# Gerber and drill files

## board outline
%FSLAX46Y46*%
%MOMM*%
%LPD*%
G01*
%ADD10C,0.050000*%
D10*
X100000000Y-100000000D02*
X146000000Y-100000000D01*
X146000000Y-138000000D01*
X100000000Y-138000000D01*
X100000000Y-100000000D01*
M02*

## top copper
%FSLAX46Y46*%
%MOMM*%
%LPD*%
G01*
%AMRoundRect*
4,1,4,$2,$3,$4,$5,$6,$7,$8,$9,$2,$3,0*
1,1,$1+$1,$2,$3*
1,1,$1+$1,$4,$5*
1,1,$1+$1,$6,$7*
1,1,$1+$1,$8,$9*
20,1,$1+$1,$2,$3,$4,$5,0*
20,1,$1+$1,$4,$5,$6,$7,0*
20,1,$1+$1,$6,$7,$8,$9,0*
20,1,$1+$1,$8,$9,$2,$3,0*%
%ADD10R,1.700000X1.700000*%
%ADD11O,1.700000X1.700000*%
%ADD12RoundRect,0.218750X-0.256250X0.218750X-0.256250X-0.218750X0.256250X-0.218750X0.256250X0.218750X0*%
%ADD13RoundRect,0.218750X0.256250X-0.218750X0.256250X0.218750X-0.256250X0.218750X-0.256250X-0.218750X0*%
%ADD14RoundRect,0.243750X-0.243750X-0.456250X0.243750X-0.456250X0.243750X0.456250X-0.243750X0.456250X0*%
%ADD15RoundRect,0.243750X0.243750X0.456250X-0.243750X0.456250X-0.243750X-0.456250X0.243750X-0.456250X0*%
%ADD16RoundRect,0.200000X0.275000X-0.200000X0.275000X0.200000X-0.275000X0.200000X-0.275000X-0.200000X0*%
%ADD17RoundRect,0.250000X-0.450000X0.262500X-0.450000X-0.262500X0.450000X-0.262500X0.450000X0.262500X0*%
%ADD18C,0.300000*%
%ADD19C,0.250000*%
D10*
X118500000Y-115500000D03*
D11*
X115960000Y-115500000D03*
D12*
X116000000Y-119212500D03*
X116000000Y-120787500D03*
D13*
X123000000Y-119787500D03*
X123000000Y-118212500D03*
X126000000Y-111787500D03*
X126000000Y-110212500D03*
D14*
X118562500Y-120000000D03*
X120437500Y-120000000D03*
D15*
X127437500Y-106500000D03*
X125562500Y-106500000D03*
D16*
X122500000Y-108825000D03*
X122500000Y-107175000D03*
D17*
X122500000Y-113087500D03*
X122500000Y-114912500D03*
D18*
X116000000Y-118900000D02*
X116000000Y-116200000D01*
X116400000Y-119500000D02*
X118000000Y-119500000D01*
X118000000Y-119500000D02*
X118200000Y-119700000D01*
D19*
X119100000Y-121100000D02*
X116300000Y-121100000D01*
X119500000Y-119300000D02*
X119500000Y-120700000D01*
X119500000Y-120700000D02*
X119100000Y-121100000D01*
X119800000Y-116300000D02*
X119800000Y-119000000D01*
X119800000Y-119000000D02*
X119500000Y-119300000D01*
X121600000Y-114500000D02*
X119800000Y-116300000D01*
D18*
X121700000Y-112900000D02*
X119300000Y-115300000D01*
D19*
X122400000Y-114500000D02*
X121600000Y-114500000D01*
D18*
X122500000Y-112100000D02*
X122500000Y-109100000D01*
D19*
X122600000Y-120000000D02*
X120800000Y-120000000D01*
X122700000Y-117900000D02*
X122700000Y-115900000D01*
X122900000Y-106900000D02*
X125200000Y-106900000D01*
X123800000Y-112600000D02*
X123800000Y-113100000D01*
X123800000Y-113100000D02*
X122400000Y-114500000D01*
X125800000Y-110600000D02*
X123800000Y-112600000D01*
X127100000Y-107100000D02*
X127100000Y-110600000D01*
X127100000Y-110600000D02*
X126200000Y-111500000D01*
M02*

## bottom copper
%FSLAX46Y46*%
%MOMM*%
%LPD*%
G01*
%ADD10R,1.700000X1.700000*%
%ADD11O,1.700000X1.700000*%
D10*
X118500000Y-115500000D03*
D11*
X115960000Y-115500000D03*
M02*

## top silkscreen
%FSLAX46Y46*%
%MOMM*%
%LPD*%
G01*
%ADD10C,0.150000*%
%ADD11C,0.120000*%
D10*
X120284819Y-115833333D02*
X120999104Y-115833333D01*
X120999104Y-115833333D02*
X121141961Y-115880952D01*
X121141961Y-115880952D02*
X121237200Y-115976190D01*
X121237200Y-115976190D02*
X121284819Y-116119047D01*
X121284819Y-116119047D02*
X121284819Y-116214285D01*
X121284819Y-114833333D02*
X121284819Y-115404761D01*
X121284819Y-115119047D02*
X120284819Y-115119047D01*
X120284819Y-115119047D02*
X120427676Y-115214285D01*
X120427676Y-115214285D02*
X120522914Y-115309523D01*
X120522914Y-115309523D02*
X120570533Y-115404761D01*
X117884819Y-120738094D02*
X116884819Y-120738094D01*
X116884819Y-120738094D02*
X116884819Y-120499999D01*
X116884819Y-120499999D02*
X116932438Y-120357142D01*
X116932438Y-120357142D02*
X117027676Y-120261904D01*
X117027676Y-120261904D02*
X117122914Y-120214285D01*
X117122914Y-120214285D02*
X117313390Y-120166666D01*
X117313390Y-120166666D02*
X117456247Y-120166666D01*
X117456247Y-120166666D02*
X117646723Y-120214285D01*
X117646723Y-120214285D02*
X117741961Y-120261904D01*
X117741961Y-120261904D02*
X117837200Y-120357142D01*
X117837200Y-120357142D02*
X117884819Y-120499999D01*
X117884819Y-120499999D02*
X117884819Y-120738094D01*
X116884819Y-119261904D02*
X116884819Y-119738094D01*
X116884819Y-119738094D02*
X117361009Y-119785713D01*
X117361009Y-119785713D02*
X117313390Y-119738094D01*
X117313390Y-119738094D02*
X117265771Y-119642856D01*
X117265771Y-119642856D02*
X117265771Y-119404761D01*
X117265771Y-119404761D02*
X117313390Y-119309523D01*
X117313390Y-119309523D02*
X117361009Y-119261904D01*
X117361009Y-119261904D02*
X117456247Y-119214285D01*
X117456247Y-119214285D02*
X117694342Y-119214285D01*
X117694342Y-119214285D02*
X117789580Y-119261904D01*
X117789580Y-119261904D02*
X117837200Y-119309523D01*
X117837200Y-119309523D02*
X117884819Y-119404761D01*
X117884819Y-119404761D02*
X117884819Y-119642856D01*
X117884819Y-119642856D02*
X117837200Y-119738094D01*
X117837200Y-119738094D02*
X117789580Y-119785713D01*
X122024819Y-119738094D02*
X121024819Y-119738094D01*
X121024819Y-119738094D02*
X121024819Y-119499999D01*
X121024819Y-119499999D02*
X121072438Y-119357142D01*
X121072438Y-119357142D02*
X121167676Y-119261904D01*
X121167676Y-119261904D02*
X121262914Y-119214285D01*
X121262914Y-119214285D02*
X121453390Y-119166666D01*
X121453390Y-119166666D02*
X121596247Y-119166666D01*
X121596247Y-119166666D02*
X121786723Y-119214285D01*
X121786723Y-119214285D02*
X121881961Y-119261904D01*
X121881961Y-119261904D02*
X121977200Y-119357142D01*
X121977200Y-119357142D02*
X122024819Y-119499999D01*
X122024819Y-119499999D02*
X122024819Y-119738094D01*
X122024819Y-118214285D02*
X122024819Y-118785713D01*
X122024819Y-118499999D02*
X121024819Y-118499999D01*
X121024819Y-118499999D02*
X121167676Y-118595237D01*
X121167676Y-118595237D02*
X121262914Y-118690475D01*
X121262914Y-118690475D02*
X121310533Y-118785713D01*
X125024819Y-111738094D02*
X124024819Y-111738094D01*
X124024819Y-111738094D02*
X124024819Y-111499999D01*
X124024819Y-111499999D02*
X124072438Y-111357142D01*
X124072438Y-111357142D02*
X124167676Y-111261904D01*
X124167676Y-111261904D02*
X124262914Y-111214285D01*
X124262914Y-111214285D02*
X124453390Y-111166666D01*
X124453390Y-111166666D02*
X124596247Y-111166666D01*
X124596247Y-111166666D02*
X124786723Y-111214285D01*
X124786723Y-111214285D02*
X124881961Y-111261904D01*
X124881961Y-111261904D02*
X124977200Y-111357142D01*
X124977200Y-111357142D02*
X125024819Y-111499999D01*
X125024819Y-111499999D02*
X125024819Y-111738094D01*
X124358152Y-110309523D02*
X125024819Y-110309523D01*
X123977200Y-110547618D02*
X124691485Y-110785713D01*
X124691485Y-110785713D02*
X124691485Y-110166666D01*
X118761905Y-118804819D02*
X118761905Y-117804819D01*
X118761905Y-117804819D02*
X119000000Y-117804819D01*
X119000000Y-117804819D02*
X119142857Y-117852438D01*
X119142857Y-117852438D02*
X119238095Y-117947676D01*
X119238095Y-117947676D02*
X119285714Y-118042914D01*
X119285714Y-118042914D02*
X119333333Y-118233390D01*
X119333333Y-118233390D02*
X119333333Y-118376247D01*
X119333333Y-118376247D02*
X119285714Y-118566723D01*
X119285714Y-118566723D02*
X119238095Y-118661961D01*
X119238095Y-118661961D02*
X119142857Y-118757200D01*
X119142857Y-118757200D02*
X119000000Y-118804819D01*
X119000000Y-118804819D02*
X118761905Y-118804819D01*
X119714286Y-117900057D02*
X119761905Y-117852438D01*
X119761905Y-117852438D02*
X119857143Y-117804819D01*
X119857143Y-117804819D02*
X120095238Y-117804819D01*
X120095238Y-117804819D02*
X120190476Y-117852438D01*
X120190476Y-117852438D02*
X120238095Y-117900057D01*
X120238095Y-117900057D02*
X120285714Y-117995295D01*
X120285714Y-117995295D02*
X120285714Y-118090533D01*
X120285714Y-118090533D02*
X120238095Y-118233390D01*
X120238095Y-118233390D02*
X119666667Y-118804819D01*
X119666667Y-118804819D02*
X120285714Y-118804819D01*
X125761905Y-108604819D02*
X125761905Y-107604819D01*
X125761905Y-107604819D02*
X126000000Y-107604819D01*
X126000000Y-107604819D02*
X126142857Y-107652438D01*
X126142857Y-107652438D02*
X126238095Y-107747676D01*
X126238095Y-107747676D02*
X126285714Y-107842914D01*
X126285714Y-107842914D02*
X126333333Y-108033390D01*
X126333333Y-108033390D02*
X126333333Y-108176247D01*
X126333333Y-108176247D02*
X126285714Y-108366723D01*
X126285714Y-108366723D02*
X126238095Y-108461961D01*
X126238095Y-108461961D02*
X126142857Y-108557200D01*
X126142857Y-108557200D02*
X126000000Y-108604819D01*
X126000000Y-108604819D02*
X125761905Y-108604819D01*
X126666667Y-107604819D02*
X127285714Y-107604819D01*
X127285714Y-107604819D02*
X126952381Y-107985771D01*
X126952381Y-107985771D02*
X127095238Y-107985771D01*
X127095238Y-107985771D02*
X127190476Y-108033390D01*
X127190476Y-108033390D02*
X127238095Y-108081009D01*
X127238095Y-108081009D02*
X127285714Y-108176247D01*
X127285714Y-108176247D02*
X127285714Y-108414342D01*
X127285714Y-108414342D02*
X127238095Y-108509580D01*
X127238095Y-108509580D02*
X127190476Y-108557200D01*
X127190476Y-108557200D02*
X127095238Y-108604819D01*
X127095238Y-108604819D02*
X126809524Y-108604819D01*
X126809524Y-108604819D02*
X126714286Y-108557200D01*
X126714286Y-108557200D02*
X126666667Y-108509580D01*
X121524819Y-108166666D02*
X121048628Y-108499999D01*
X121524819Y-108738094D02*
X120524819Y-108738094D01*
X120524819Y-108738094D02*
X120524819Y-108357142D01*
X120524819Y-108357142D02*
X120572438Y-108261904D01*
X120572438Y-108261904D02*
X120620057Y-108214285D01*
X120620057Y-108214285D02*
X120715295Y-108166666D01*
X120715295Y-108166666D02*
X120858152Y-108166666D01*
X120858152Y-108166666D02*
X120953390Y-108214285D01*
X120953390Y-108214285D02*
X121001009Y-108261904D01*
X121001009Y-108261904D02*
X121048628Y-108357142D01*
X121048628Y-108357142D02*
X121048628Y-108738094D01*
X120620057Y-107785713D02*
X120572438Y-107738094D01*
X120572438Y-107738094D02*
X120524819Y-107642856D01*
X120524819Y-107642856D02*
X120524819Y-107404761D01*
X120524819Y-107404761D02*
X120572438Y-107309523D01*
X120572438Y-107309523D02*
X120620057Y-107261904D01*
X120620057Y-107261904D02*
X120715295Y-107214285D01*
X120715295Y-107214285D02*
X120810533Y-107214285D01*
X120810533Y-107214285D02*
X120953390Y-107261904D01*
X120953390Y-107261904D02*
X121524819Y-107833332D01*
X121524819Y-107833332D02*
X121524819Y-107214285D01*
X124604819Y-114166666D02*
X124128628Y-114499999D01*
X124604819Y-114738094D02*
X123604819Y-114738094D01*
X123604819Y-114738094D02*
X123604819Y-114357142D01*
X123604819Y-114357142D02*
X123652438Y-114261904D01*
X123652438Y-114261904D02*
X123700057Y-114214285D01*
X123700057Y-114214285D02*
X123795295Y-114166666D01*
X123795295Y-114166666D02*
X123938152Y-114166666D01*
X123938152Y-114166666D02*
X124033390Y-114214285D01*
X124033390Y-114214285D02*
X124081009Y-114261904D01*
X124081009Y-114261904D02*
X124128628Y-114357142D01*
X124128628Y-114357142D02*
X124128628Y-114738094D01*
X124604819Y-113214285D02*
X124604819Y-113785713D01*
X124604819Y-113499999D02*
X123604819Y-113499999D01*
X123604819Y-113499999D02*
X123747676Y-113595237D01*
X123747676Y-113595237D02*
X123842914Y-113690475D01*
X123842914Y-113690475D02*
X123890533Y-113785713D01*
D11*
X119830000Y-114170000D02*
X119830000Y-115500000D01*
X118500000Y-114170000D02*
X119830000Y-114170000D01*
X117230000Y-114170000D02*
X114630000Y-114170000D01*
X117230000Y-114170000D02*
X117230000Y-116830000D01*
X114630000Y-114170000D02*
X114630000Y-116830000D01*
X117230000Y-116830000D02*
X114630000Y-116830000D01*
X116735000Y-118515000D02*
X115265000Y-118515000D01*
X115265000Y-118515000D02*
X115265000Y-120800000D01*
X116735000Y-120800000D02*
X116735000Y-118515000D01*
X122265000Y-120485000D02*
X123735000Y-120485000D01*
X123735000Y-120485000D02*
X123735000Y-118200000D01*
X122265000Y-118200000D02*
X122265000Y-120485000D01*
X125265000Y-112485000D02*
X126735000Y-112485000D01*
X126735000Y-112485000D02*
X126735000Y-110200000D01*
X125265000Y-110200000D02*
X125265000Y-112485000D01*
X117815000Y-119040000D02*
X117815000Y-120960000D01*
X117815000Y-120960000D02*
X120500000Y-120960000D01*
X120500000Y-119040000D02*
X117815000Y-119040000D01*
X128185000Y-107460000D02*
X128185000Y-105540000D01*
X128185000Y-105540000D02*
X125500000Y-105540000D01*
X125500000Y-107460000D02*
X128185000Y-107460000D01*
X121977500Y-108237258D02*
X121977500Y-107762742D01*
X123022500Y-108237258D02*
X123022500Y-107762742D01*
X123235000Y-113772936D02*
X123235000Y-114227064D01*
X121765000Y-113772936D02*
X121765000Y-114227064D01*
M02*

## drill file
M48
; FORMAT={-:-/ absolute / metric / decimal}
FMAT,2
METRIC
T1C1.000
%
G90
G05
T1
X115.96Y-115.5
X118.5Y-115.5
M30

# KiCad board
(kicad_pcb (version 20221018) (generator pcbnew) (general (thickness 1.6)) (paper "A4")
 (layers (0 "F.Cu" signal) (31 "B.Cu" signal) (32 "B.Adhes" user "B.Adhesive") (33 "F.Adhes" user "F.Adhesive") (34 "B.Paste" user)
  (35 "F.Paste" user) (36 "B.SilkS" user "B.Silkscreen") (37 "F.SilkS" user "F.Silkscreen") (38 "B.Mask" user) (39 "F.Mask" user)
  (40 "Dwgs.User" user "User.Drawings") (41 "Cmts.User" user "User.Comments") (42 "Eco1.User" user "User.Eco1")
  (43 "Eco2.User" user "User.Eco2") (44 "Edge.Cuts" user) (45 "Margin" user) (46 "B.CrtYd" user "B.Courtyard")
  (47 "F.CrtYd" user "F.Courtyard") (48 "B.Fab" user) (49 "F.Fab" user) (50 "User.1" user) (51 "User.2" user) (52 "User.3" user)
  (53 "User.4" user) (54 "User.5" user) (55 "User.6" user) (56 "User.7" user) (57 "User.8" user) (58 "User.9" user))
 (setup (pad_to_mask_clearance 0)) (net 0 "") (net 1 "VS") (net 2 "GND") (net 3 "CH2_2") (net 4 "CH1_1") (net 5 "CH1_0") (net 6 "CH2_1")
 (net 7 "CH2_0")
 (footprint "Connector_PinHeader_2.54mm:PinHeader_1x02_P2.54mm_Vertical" (layer "F.Cu") (at 118.5 115.5 -90)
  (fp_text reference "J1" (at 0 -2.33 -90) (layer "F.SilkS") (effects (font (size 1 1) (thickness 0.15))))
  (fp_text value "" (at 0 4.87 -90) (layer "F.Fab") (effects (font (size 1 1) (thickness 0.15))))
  (fp_line (start -1.33 -1.33) (end 0 -1.33) (stroke (width 0.12) (type solid)) (layer "F.SilkS"))
  (fp_line (start -1.33 0) (end -1.33 -1.33) (stroke (width 0.12) (type solid)) (layer "F.SilkS"))
  (fp_line (start -1.33 1.27) (end -1.33 3.87) (stroke (width 0.12) (type solid)) (layer "F.SilkS"))
  (fp_line (start -1.33 1.27) (end 1.33 1.27) (stroke (width 0.12) (type solid)) (layer "F.SilkS"))
  (fp_line (start -1.33 3.87) (end 1.33 3.87) (stroke (width 0.12) (type solid)) (layer "F.SilkS"))
  (fp_line (start 1.33 1.27) (end 1.33 3.87) (stroke (width 0.12) (type solid)) (layer "F.SilkS"))
  (pad "1" thru_hole rect (at 0 0 270) (size 1.7 1.7) (drill 1) (layers "*.Cu" "*.Mask") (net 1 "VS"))
  (pad "2" thru_hole oval (at 0 2.54 270) (size 1.7 1.7) (drill 1) (layers "*.Cu" "*.Mask") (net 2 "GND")))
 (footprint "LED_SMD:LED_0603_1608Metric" (layer "F.Cu") (at 116 120 -90)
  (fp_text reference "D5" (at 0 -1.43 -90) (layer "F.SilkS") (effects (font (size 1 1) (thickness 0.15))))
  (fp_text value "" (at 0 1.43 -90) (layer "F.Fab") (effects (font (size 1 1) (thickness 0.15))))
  (fp_line (start -1.485 -0.735) (end -1.485 0.735) (stroke (width 0.12) (type solid)) (layer "F.SilkS"))
  (fp_line (start -1.485 0.735) (end 0.8 0.735) (stroke (width 0.12) (type solid)) (layer "F.SilkS"))
  (fp_line (start 0.8 -0.735) (end -1.485 -0.735) (stroke (width 0.12) (type solid)) (layer "F.SilkS"))
  (pad "1" smd roundrect (at -0.7875 0 270) (size 0.875 0.95) (layers "F.Cu" "F.Paste" "F.Mask") (roundrect_rratio 0.25) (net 2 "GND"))
  (pad "2" smd roundrect (at 0.7875 0 270) (size 0.875 0.95) (layers "F.Cu" "F.Paste" "F.Mask") (roundrect_rratio 0.25) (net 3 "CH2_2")))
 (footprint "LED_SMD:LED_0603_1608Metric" (layer "F.Cu") (at 123 119 90)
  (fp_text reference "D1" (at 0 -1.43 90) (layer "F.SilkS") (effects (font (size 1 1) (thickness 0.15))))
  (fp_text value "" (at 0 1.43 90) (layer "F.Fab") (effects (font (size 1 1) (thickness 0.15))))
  (fp_line (start -1.485 -0.735) (end -1.485 0.735) (stroke (width 0.12) (type solid)) (layer "F.SilkS"))
  (fp_line (start -1.485 0.735) (end 0.8 0.735) (stroke (width 0.12) (type solid)) (layer "F.SilkS"))
  (fp_line (start 0.8 -0.735) (end -1.485 -0.735) (stroke (width 0.12) (type solid)) (layer "F.SilkS"))
  (pad "1" smd roundrect (at -0.7875 0 90) (size 0.875 0.95) (layers "F.Cu" "F.Paste" "F.Mask") (roundrect_rratio 0.25) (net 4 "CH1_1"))
  (pad "2" smd roundrect (at 0.7875 0 90) (size 0.875 0.95) (layers "F.Cu" "F.Paste" "F.Mask") (roundrect_rratio 0.25) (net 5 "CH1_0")))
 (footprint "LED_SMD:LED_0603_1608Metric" (layer "F.Cu") (at 126 111 90)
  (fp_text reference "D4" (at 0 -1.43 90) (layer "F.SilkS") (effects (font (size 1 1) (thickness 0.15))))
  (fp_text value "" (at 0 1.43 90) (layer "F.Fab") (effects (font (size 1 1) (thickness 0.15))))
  (fp_line (start -1.485 -0.735) (end -1.485 0.735) (stroke (width 0.12) (type solid)) (layer "F.SilkS"))
  (fp_line (start -1.485 0.735) (end 0.8 0.735) (stroke (width 0.12) (type solid)) (layer "F.SilkS"))
  (fp_line (start 0.8 -0.735) (end -1.485 -0.735) (stroke (width 0.12) (type solid)) (layer "F.SilkS"))
  (pad "1" smd roundrect (at -0.7875 0 90) (size 0.875 0.95) (layers "F.Cu" "F.Paste" "F.Mask") (roundrect_rratio 0.25) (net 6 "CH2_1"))
  (pad "2" smd roundrect (at 0.7875 0 90) (size 0.875 0.95) (layers "F.Cu" "F.Paste" "F.Mask") (roundrect_rratio 0.25) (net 3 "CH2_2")))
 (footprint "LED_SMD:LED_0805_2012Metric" (layer "F.Cu") (at 119.5 120)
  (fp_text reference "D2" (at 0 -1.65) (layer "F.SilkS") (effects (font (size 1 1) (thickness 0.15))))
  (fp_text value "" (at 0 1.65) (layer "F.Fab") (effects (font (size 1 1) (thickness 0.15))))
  (fp_line (start -1.685 -0.96) (end -1.685 0.96) (stroke (width 0.12) (type solid)) (layer "F.SilkS"))
  (fp_line (start -1.685 0.96) (end 1 0.96) (stroke (width 0.12) (type solid)) (layer "F.SilkS"))
  (fp_line (start 1 -0.96) (end -1.685 -0.96) (stroke (width 0.12) (type solid)) (layer "F.SilkS"))
  (pad "1" smd roundrect (at -0.9375 0) (size 0.975 1.4) (layers "F.Cu" "F.Paste" "F.Mask") (roundrect_rratio 0.25) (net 2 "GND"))
  (pad "2" smd roundrect (at 0.9375 0) (size 0.975 1.4) (layers "F.Cu" "F.Paste" "F.Mask") (roundrect_rratio 0.25) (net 4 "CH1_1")))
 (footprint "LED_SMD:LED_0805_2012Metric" (layer "F.Cu") (at 126.5 106.5 180)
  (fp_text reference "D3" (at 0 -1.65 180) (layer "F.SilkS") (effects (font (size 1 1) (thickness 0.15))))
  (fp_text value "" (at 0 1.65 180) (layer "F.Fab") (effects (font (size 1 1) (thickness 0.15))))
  (fp_line (start -1.685 -0.96) (end -1.685 0.96) (stroke (width 0.12) (type solid)) (layer "F.SilkS"))
  (fp_line (start -1.685 0.96) (end 1 0.96) (stroke (width 0.12) (type solid)) (layer "F.SilkS"))
  (fp_line (start 1 -0.96) (end -1.685 -0.96) (stroke (width 0.12) (type solid)) (layer "F.SilkS"))
  (pad "1" smd roundrect (at -0.9375 0 180) (size 0.975 1.4) (layers "F.Cu" "F.Paste" "F.Mask") (roundrect_rratio 0.25) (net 6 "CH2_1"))
  (pad "2" smd roundrect (at 0.9375 0 180) (size 0.975 1.4) (layers "F.Cu" "F.Paste" "F.Mask") (roundrect_rratio 0.25) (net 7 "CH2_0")))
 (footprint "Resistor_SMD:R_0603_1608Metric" (layer "F.Cu") (at 122.5 108 90)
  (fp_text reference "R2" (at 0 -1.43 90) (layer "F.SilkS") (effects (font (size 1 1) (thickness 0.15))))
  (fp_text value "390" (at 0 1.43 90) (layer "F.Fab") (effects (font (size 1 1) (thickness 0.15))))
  (fp_line (start -0.237258 -0.5225) (end 0.237258 -0.5225) (stroke (width 0.12) (type solid)) (layer "F.SilkS"))
  (fp_line (start -0.237258 0.5225) (end 0.237258 0.5225) (stroke (width 0.12) (type solid)) (layer "F.SilkS"))
  (pad "1" smd roundrect (at -0.825 0 90) (size 0.8 0.95) (layers "F.Cu" "F.Paste" "F.Mask") (roundrect_rratio 0.25) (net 1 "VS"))
  (pad "2" smd roundrect (at 0.825 0 90) (size 0.8 0.95) (layers "F.Cu" "F.Paste" "F.Mask") (roundrect_rratio 0.25) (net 7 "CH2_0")))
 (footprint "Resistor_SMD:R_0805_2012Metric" (layer "F.Cu") (at 122.5 114 -90)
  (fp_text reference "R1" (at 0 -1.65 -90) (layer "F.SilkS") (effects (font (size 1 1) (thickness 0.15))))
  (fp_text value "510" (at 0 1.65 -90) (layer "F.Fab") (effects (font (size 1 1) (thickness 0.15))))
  (fp_line (start -0.227064 -0.735) (end 0.227064 -0.735) (stroke (width 0.12) (type solid)) (layer "F.SilkS"))
  (fp_line (start -0.227064 0.735) (end 0.227064 0.735) (stroke (width 0.12) (type solid)) (layer "F.SilkS"))
  (pad "1" smd roundrect (at -0.9125 0 270) (size 1.025 1.4) (layers "F.Cu" "F.Paste" "F.Mask") (roundrect_rratio 0.243902) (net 1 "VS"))
  (pad "2" smd roundrect (at 0.9125 0 270) (size 1.025 1.4) (layers "F.Cu" "F.Paste" "F.Mask") (roundrect_rratio 0.243902) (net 5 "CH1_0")))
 (gr_rect (start 100 100) (end 146 138) (stroke (width 0.05) (type default)) (fill none) (layer "Edge.Cuts"))
 (segment (start 116 118.9) (end 116 116.2) (width 0.3) (layer "F.Cu") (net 2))
 (segment (start 116.4 119.5) (end 118 119.5) (width 0.3) (layer "F.Cu") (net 2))
 (segment (start 118 119.5) (end 118.2 119.7) (width 0.3) (layer "F.Cu") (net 2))
 (segment (start 119.1 121.1) (end 116.3 121.1) (width 0.25) (layer "F.Cu") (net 3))
 (segment (start 119.5 119.3) (end 119.5 120.7) (width 0.25) (layer "F.Cu") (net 3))
 (segment (start 119.5 120.7) (end 119.1 121.1) (width 0.25) (layer "F.Cu") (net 3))
 (segment (start 119.8 116.3) (end 119.8 119) (width 0.25) (layer "F.Cu") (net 3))
 (segment (start 119.8 119) (end 119.5 119.3) (width 0.25) (layer "F.Cu") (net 3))
 (segment (start 121.6 114.5) (end 119.8 116.3) (width 0.25) (layer "F.Cu") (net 3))
 (segment (start 121.7 112.9) (end 119.3 115.3) (width 0.3) (layer "F.Cu") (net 1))
 (segment (start 122.4 114.5) (end 121.6 114.5) (width 0.25) (layer "F.Cu") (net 3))
 (segment (start 122.5 112.1) (end 122.5 109.1) (width 0.3) (layer "F.Cu") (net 1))
 (segment (start 122.6 120) (end 120.8 120) (width 0.25) (layer "F.Cu") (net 4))
 (segment (start 122.7 117.9) (end 122.7 115.9) (width 0.25) (layer "F.Cu") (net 5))
 (segment (start 122.9 106.9) (end 125.2 106.9) (width 0.25) (layer "F.Cu") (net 7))
 (segment (start 123.8 112.6) (end 123.8 113.1) (width 0.25) (layer "F.Cu") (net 3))
 (segment (start 123.8 113.1) (end 122.4 114.5) (width 0.25) (layer "F.Cu") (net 3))
 (segment (start 125.8 110.6) (end 123.8 112.6) (width 0.25) (layer "F.Cu") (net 3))
 (segment (start 127.1 107.1) (end 127.1 110.6) (width 0.25) (layer "F.Cu") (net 6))
 (segment (start 127.1 110.6) (end 126.2 111.5) (width 0.25) (layer "F.Cu") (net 6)))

